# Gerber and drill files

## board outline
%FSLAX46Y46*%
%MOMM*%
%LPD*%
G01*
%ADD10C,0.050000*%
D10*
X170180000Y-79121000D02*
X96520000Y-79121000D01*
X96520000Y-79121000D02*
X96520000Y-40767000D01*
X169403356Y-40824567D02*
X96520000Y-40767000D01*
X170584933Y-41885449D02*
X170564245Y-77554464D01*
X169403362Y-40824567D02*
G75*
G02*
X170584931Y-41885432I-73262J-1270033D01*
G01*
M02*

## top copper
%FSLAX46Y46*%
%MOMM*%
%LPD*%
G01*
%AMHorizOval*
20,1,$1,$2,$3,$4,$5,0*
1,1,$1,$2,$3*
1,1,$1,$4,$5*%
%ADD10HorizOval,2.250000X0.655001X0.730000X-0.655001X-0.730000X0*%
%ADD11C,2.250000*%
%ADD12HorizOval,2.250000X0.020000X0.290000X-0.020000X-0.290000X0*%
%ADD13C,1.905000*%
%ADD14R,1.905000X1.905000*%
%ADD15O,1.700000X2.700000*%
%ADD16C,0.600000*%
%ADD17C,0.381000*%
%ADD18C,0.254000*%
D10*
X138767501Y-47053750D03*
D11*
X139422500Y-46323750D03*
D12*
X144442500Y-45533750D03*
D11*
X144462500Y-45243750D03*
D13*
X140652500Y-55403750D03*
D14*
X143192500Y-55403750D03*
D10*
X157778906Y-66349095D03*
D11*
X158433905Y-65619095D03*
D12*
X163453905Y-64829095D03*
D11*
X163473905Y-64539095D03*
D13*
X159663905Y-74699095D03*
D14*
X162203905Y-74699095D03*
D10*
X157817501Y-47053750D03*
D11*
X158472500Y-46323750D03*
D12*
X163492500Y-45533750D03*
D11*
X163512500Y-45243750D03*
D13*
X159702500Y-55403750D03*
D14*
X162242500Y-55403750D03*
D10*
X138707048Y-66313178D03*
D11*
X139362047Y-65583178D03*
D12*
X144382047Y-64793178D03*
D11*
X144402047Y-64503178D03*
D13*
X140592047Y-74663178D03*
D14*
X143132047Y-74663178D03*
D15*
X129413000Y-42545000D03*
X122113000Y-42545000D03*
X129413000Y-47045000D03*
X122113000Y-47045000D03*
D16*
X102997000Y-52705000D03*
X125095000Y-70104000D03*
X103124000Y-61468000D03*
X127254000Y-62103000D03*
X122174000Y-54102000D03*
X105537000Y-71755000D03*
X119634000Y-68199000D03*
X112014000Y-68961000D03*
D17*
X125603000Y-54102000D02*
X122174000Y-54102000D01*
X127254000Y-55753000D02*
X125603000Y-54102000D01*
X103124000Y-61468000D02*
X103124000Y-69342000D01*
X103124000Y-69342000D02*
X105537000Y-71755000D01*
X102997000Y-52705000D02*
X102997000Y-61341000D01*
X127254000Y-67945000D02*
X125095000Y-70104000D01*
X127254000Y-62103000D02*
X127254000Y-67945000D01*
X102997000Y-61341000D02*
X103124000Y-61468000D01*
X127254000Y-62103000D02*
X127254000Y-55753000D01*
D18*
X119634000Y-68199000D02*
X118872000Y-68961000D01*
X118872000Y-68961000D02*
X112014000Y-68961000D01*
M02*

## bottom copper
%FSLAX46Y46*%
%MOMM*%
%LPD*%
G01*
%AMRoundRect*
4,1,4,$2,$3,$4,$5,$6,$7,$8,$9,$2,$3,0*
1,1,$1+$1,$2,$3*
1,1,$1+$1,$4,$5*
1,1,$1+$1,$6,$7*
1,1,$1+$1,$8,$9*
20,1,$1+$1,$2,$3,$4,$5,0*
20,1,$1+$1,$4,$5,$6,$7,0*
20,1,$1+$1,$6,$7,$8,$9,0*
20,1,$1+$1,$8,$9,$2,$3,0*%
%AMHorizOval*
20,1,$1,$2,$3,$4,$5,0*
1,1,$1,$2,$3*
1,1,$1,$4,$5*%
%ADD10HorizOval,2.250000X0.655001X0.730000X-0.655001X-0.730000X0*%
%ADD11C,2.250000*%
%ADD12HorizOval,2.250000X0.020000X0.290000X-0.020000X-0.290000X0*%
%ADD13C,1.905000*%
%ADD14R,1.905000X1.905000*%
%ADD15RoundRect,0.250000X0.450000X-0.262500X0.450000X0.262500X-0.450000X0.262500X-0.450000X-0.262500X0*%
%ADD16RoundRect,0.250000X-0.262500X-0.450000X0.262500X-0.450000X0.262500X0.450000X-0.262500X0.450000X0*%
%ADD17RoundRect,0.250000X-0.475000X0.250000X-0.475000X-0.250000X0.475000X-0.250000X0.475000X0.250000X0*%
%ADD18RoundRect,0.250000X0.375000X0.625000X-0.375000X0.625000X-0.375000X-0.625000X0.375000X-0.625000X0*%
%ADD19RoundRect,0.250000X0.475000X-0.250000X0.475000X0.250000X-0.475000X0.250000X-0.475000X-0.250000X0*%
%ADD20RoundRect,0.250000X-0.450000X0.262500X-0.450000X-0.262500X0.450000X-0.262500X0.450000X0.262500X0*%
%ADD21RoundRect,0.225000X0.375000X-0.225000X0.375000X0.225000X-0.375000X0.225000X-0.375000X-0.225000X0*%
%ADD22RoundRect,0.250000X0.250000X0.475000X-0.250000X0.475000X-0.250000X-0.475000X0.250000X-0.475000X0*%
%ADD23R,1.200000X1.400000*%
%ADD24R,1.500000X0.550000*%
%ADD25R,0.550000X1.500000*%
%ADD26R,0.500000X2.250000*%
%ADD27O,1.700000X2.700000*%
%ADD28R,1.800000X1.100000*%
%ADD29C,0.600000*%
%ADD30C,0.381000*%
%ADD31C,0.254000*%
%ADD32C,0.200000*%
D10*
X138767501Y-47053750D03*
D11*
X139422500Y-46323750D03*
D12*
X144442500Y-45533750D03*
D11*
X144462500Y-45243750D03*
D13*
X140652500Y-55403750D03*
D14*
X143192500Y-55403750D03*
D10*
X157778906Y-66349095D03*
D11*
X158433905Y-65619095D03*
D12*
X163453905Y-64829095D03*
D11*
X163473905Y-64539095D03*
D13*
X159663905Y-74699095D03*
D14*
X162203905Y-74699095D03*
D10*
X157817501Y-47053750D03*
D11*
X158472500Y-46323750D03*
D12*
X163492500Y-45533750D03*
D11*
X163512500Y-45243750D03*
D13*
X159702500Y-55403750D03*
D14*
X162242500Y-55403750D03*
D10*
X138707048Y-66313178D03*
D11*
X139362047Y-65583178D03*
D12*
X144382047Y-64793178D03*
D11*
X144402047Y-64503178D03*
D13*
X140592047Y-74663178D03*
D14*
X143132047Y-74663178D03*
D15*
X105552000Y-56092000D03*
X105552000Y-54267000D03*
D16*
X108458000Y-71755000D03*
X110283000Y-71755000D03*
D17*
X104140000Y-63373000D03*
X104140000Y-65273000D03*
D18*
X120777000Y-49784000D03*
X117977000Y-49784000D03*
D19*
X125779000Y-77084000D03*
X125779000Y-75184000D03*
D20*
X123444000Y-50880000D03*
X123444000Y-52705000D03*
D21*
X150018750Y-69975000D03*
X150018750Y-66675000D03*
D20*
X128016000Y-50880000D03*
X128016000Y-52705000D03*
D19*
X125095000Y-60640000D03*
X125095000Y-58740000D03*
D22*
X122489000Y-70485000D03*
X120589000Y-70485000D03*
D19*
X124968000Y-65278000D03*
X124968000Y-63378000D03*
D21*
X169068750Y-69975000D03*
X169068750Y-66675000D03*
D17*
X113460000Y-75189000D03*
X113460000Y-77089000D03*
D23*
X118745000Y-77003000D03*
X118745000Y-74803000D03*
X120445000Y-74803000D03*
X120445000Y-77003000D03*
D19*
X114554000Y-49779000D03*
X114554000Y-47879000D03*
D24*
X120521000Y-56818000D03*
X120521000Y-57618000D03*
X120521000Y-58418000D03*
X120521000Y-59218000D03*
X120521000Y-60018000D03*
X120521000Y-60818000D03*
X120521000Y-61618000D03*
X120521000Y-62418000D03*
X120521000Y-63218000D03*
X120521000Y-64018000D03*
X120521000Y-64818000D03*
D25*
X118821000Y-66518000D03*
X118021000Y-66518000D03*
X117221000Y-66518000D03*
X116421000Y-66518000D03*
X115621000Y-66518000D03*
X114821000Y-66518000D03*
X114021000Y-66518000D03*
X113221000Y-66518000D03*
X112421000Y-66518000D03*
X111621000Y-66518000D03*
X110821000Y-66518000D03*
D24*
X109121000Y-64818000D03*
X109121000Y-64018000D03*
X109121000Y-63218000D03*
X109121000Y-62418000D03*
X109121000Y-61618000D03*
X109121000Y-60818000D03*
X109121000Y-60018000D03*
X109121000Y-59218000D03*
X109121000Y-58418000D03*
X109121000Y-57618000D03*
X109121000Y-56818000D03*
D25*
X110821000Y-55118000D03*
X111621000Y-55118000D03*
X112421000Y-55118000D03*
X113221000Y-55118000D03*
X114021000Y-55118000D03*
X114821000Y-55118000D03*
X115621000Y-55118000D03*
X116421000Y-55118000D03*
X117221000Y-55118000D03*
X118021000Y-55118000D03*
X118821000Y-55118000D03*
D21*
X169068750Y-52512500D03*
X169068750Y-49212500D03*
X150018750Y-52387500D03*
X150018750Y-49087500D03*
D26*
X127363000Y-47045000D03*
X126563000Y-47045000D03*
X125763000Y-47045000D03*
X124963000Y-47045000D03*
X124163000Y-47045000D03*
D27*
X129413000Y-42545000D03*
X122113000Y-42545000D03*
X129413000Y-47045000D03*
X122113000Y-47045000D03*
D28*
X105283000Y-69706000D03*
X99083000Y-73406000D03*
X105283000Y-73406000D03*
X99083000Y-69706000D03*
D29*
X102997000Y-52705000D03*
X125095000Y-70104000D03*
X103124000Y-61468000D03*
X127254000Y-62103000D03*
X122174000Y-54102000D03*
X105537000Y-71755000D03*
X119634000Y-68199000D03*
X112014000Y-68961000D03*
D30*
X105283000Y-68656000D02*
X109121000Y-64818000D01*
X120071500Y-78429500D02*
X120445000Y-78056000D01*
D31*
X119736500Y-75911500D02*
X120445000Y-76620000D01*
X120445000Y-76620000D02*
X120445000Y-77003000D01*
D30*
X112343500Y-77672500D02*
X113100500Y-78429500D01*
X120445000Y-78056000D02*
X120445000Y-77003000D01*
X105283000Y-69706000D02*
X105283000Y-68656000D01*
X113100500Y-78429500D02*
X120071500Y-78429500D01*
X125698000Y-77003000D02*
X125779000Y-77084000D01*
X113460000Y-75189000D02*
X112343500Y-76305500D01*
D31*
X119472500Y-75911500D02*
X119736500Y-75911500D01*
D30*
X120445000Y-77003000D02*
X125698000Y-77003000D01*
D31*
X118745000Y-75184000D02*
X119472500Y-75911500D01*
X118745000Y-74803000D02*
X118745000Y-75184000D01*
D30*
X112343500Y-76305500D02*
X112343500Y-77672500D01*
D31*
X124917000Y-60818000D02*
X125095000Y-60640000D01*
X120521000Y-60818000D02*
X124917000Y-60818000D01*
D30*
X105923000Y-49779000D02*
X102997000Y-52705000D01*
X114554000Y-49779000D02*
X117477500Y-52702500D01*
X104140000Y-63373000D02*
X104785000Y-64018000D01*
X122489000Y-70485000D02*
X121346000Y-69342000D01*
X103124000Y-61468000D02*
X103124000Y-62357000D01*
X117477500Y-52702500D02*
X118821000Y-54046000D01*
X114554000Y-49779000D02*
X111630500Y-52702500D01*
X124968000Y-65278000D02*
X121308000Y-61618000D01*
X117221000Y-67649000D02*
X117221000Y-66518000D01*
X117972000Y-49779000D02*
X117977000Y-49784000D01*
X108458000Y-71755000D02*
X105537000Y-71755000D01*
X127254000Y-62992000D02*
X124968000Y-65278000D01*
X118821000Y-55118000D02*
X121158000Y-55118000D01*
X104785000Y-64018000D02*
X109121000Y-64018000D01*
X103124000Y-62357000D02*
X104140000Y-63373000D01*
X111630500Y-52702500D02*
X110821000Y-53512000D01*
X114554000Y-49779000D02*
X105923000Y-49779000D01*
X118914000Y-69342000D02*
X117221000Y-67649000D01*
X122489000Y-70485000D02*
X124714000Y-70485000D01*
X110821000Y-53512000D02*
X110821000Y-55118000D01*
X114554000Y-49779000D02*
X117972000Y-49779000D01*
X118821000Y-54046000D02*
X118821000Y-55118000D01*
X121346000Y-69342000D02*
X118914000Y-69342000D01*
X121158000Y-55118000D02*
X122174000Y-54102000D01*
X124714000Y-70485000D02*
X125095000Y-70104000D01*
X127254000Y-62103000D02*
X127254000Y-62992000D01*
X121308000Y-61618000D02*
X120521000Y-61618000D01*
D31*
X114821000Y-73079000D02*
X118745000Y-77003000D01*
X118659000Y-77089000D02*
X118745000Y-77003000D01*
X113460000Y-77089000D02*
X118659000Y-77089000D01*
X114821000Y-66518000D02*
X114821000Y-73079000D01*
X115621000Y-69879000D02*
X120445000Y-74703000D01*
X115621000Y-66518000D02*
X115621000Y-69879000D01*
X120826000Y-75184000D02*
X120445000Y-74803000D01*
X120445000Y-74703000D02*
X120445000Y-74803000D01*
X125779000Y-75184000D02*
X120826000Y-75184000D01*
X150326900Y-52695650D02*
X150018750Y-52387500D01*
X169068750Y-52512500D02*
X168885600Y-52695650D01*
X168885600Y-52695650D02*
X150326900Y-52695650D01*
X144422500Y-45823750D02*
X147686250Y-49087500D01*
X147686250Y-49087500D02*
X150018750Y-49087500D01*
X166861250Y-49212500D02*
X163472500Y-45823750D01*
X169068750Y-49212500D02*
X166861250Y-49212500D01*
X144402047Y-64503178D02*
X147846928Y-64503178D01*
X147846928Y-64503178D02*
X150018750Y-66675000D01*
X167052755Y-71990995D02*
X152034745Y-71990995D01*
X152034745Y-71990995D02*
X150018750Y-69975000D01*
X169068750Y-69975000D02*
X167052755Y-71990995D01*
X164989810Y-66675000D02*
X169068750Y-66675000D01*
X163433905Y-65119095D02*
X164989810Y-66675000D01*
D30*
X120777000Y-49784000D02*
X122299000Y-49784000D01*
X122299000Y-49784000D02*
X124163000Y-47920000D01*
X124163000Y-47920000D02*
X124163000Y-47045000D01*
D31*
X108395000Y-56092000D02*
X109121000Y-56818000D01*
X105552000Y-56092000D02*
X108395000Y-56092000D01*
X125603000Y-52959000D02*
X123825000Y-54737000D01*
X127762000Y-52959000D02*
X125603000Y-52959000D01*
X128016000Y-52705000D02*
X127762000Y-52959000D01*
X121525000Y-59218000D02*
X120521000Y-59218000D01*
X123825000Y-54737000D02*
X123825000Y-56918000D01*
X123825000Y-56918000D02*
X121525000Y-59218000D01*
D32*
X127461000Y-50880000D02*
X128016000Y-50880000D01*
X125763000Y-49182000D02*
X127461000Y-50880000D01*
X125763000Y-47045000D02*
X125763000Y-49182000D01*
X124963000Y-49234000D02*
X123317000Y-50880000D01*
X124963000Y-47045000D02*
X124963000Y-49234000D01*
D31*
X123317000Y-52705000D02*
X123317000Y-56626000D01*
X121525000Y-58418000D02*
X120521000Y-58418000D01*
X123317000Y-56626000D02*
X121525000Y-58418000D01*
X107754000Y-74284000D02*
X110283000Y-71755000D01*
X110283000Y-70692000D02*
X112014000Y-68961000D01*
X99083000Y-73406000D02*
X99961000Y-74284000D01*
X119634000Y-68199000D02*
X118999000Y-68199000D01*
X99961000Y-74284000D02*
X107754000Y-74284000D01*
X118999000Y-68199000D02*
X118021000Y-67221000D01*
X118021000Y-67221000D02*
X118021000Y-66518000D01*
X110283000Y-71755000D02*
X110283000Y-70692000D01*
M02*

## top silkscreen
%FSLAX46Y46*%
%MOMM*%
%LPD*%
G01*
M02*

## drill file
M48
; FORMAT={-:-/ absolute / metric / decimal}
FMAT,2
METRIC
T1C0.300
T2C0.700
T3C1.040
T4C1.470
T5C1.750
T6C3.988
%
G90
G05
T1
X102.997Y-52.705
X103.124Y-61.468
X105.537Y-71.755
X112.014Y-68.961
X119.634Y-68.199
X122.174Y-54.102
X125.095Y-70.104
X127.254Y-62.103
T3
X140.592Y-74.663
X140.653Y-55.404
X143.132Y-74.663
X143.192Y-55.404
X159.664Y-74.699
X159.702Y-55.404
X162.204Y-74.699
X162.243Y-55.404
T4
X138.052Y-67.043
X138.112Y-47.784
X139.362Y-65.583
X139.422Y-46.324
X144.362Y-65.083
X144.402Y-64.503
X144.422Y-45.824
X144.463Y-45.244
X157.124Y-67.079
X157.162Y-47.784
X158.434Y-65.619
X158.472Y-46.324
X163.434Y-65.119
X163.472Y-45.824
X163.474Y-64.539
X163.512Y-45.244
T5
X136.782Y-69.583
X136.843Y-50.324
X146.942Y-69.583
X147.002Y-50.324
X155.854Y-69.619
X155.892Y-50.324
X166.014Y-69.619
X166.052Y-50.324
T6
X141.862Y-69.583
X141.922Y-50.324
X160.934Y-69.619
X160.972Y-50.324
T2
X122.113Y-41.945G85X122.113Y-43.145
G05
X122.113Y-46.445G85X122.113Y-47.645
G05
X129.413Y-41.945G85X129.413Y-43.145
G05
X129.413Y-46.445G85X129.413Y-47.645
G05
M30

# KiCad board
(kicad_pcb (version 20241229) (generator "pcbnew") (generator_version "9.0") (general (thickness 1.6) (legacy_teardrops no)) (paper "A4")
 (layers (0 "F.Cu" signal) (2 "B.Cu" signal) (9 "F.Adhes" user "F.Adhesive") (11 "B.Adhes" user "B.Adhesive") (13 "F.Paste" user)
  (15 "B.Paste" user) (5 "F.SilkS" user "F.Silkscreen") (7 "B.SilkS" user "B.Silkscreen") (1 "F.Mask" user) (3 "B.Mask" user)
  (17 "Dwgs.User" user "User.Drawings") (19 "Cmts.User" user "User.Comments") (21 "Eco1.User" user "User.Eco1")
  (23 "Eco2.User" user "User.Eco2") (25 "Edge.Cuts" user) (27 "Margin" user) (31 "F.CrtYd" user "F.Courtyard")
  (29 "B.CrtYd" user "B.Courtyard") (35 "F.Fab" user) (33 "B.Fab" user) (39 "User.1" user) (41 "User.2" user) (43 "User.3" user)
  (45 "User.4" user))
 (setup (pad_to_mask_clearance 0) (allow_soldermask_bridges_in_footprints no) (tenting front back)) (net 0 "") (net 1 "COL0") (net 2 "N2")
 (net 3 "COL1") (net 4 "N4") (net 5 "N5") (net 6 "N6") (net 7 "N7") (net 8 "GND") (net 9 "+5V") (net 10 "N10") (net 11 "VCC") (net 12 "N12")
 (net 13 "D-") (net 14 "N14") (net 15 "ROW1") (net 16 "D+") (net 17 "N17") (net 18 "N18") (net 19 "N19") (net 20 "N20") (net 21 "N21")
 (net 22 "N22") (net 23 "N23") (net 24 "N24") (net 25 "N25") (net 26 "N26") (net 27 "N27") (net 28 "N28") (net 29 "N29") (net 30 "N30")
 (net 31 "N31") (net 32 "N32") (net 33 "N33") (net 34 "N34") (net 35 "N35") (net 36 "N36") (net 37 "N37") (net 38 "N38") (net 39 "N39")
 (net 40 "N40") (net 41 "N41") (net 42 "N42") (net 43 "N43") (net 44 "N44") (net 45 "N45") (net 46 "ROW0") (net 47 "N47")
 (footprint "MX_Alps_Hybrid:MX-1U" (layer "F.Cu") (at 141.9225 50.32375)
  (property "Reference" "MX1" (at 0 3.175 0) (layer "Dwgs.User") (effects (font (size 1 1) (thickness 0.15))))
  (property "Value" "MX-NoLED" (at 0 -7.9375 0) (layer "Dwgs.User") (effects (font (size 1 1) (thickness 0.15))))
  (pad "" np_thru_hole circle (at -5.08 0 48.0996) (size 1.75 1.75) (drill 1.75) (layers "*.Cu" "*.Mask"))
  (pad "" np_thru_hole circle (at 0 0) (size 3.9878 3.9878) (drill 3.9878) (layers "*.Cu" "*.Mask"))
  (pad "" np_thru_hole circle (at 5.08 0 48.0996) (size 1.75 1.75) (drill 1.75) (layers "*.Cu" "*.Mask"))
  (pad "1" thru_hole oval (at -3.81 -2.54 48.0996) (size 4.211556 2.25) (drill 1.47 (offset 0.980778 0)) (layers "*.Cu" "B.Mask")
   (remove_unused_layers no) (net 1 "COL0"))
  (pad "1" thru_hole circle (at -2.5 -4) (size 2.25 2.25) (drill 1.47) (layers "*.Cu" "B.Mask") (remove_unused_layers no) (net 1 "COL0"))
  (pad "2" thru_hole oval (at 2.5 -4.5 86.0548) (size 2.831378 2.25) (drill 1.47 (offset 0.290689 0)) (layers "*.Cu" "B.Mask")
   (remove_unused_layers no) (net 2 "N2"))
  (pad "2" thru_hole circle (at 2.54 -5.08) (size 2.25 2.25) (drill 1.47) (layers "*.Cu" "B.Mask") (remove_unused_layers no) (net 2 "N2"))
  (pad "3" thru_hole circle (at -1.27 5.08) (size 1.905 1.905) (drill 1.04) (layers "*.Cu" "B.Mask") (remove_unused_layers no))
  (pad "4" thru_hole rect (at 1.27 5.08) (size 1.905 1.905) (drill 1.04) (layers "*.Cu" "B.Mask") (remove_unused_layers no)))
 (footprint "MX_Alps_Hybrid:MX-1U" (layer "F.Cu") (at 160.933905 69.619095)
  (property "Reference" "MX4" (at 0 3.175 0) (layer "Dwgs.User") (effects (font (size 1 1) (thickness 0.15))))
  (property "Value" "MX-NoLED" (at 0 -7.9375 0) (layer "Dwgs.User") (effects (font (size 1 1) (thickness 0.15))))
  (pad "" np_thru_hole circle (at -5.08 0 48.0996) (size 1.75 1.75) (drill 1.75) (layers "*.Cu" "*.Mask"))
  (pad "" np_thru_hole circle (at 0 0) (size 3.9878 3.9878) (drill 3.9878) (layers "*.Cu" "*.Mask"))
  (pad "" np_thru_hole circle (at 5.08 0 48.0996) (size 1.75 1.75) (drill 1.75) (layers "*.Cu" "*.Mask"))
  (pad "1" thru_hole oval (at -3.81 -2.54 48.0996) (size 4.211556 2.25) (drill 1.47 (offset 0.980778 0)) (layers "*.Cu" "B.Mask")
   (remove_unused_layers no) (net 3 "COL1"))
  (pad "1" thru_hole circle (at -2.5 -4) (size 2.25 2.25) (drill 1.47) (layers "*.Cu" "B.Mask") (remove_unused_layers no) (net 3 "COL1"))
  (pad "2" thru_hole oval (at 2.5 -4.5 86.0548) (size 2.831378 2.25) (drill 1.47 (offset 0.290689 0)) (layers "*.Cu" "B.Mask")
   (remove_unused_layers no) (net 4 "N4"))
  (pad "2" thru_hole circle (at 2.54 -5.08) (size 2.25 2.25) (drill 1.47) (layers "*.Cu" "B.Mask") (remove_unused_layers no) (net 4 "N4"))
  (pad "3" thru_hole circle (at -1.27 5.08) (size 1.905 1.905) (drill 1.04) (layers "*.Cu" "B.Mask") (remove_unused_layers no))
  (pad "4" thru_hole rect (at 1.27 5.08) (size 1.905 1.905) (drill 1.04) (layers "*.Cu" "B.Mask") (remove_unused_layers no)))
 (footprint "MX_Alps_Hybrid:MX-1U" (layer "F.Cu") (at 160.9725 50.32375)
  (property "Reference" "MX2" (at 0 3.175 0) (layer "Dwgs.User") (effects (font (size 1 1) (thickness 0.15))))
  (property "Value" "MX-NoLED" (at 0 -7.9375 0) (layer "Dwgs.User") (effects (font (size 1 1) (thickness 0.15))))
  (pad "" np_thru_hole circle (at -5.08 0 48.0996) (size 1.75 1.75) (drill 1.75) (layers "*.Cu" "*.Mask"))
  (pad "" np_thru_hole circle (at 0 0) (size 3.9878 3.9878) (drill 3.9878) (layers "*.Cu" "*.Mask"))
  (pad "" np_thru_hole circle (at 5.08 0 48.0996) (size 1.75 1.75) (drill 1.75) (layers "*.Cu" "*.Mask"))
  (pad "1" thru_hole oval (at -3.81 -2.54 48.0996) (size 4.211556 2.25) (drill 1.47 (offset 0.980778 0)) (layers "*.Cu" "B.Mask")
   (remove_unused_layers no) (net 3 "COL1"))
  (pad "1" thru_hole circle (at -2.5 -4) (size 2.25 2.25) (drill 1.47) (layers "*.Cu" "B.Mask") (remove_unused_layers no) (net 3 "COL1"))
  (pad "2" thru_hole oval (at 2.5 -4.5 86.0548) (size 2.831378 2.25) (drill 1.47 (offset 0.290689 0)) (layers "*.Cu" "B.Mask")
   (remove_unused_layers no) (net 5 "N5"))
  (pad "2" thru_hole circle (at 2.54 -5.08) (size 2.25 2.25) (drill 1.47) (layers "*.Cu" "B.Mask") (remove_unused_layers no) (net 5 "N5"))
  (pad "3" thru_hole circle (at -1.27 5.08) (size 1.905 1.905) (drill 1.04) (layers "*.Cu" "B.Mask") (remove_unused_layers no))
  (pad "4" thru_hole rect (at 1.27 5.08) (size 1.905 1.905) (drill 1.04) (layers "*.Cu" "B.Mask") (remove_unused_layers no)))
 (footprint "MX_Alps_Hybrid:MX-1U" (layer "F.Cu") (at 141.862047 69.583178)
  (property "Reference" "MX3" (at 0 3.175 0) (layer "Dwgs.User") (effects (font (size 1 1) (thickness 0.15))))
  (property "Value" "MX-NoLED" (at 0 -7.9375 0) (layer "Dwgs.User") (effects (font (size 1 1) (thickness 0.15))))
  (pad "" np_thru_hole circle (at -5.08 0 48.0996) (size 1.75 1.75) (drill 1.75) (layers "*.Cu" "*.Mask"))
  (pad "" np_thru_hole circle (at 0 0) (size 3.9878 3.9878) (drill 3.9878) (layers "*.Cu" "*.Mask"))
  (pad "" np_thru_hole circle (at 5.08 0 48.0996) (size 1.75 1.75) (drill 1.75) (layers "*.Cu" "*.Mask"))
  (pad "1" thru_hole oval (at -3.81 -2.54 48.0996) (size 4.211556 2.25) (drill 1.47 (offset 0.980778 0)) (layers "*.Cu" "B.Mask")
   (remove_unused_layers no) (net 1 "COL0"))
  (pad "1" thru_hole circle (at -2.5 -4) (size 2.25 2.25) (drill 1.47) (layers "*.Cu" "B.Mask") (remove_unused_layers no) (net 1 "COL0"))
  (pad "2" thru_hole oval (at 2.5 -4.5 86.0548) (size 2.831378 2.25) (drill 1.47 (offset 0.290689 0)) (layers "*.Cu" "B.Mask")
   (remove_unused_layers no) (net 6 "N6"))
  (pad "2" thru_hole circle (at 2.54 -5.08) (size 2.25 2.25) (drill 1.47) (layers "*.Cu" "B.Mask") (remove_unused_layers no) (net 6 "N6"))
  (pad "3" thru_hole circle (at -1.27 5.08) (size 1.905 1.905) (drill 1.04) (layers "*.Cu" "B.Mask") (remove_unused_layers no))
  (pad "4" thru_hole rect (at 1.27 5.08) (size 1.905 1.905) (drill 1.04) (layers "*.Cu" "B.Mask") (remove_unused_layers no)))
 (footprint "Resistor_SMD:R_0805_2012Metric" (layer "B.Cu") (at 105.552 55.1795 90)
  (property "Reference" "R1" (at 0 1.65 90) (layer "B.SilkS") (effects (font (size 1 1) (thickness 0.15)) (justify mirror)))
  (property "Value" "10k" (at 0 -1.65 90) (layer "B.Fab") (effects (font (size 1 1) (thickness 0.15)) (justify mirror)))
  (pad "1" smd roundrect (at -0.9125 0 90) (size 1.025 1.4) (layers "B.Cu" "B.Mask" "B.Paste") (roundrect_rratio 0.243902) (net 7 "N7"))
  (pad "2" smd roundrect (at 0.9125 0 90) (size 1.025 1.4) (layers "B.Cu" "B.Mask" "B.Paste") (roundrect_rratio 0.243902) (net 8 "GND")))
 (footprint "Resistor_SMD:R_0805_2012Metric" (layer "B.Cu") (at 109.3705 71.755)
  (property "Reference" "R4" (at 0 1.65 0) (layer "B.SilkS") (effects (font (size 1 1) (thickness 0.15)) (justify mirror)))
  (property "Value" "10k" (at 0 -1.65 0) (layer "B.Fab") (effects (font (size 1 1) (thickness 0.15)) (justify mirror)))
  (pad "1" smd roundrect (at -0.9125 0) (size 1.025 1.4) (layers "B.Cu" "B.Mask" "B.Paste") (roundrect_rratio 0.243902) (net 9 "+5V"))
  (pad "2" smd roundrect (at 0.9125 0) (size 1.025 1.4) (layers "B.Cu" "B.Mask" "B.Paste") (roundrect_rratio 0.243902) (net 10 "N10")))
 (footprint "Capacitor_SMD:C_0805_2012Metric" (layer "B.Cu") (at 104.14 64.323 -90)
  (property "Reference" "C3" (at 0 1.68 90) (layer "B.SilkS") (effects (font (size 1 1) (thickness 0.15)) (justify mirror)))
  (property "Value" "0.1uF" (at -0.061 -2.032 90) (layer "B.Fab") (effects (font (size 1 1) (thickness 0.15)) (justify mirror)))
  (pad "1" smd roundrect (at -0.95 0 270) (size 1 1.45) (layers "B.Cu" "B.Mask" "B.Paste") (roundrect_rratio 0.25) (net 9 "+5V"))
  (pad "2" smd roundrect (at 0.95 0 270) (size 1 1.45) (layers "B.Cu" "B.Mask" "B.Paste") (roundrect_rratio 0.25) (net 8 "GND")))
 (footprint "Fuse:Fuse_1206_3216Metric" (layer "B.Cu") (at 119.377 49.784 180)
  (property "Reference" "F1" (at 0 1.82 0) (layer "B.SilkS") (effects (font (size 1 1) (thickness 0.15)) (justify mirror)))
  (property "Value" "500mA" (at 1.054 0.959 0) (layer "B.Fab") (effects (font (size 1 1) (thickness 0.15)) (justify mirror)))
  (pad "1" smd roundrect (at -1.4 0 180) (size 1.25 1.75) (layers "B.Cu" "B.Mask" "B.Paste") (roundrect_rratio 0.2) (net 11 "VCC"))
  (pad "2" smd roundrect (at 1.4 0 180) (size 1.25 1.75) (layers "B.Cu" "B.Mask" "B.Paste") (roundrect_rratio 0.2) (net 9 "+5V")))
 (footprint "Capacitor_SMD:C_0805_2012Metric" (layer "B.Cu") (at 125.779 76.134 90)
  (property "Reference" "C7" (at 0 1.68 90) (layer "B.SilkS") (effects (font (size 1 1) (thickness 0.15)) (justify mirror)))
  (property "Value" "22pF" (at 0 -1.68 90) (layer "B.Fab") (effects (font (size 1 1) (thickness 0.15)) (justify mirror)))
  (pad "1" smd roundrect (at -0.95 0 90) (size 1 1.45) (layers "B.Cu" "B.Mask" "B.Paste") (roundrect_rratio 0.25) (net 8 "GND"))
  (pad "2" smd roundrect (at 0.95 0 90) (size 1 1.45) (layers "B.Cu" "B.Mask" "B.Paste") (roundrect_rratio 0.25) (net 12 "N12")))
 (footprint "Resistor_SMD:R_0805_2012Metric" (layer "B.Cu") (at 123.444 51.7925 -90)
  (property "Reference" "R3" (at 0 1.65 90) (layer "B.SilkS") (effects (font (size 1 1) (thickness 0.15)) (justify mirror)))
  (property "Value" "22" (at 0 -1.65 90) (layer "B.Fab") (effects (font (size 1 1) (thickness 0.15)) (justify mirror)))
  (pad "1" smd roundrect (at -0.9125 0 270) (size 1.025 1.4) (layers "B.Cu" "B.Mask" "B.Paste") (roundrect_rratio 0.243902) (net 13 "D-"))
  (pad "2" smd roundrect (at 0.9125 0 270) (size 1.025 1.4) (layers "B.Cu" "B.Mask" "B.Paste") (roundrect_rratio 0.243902) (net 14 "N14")))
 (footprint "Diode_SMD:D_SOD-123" (layer "B.Cu") (at 150.01875 68.325 90)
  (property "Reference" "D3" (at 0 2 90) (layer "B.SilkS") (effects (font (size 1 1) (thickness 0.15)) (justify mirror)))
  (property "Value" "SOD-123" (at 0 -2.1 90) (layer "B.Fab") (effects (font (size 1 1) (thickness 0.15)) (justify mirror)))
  (pad "1" smd roundrect (at -1.65 0 90) (size 0.9 1.2) (layers "B.Cu" "B.Mask" "B.Paste") (roundrect_rratio 0.25) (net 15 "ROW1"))
  (pad "2" smd roundrect (at 1.65 0 90) (size 0.9 1.2) (layers "B.Cu" "B.Mask" "B.Paste") (roundrect_rratio 0.25) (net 6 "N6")))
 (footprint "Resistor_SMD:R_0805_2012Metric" (layer "B.Cu") (at 128.016 51.7925 -90)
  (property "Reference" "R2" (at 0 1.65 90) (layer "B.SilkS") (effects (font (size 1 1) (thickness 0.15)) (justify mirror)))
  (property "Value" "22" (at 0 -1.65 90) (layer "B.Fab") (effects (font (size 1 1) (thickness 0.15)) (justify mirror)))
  (pad "1" smd roundrect (at -0.9125 0 270) (size 1.025 1.4) (layers "B.Cu" "B.Mask" "B.Paste") (roundrect_rratio 0.243902) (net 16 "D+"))
  (pad "2" smd roundrect (at 0.9125 0 270) (size 1.025 1.4) (layers "B.Cu" "B.Mask" "B.Paste") (roundrect_rratio 0.243902) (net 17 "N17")))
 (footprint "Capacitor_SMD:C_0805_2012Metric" (layer "B.Cu") (at 125.095 59.69 90)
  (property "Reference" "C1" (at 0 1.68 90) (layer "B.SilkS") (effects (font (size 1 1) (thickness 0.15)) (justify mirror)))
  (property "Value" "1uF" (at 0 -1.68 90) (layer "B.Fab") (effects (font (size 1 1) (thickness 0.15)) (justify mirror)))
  (pad "1" smd roundrect (at -0.95 0 90) (size 1 1.45) (layers "B.Cu" "B.Mask" "B.Paste") (roundrect_rratio 0.25) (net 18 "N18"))
  (pad "2" smd roundrect (at 0.95 0 90) (size 1 1.45) (layers "B.Cu" "B.Mask" "B.Paste") (roundrect_rratio 0.25) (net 8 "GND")))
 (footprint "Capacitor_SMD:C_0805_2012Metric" (layer "B.Cu") (at 121.539 70.485 180)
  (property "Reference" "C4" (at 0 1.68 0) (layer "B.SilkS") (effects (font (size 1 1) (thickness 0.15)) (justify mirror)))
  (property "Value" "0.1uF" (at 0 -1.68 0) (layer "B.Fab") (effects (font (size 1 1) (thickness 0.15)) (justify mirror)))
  (pad "1" smd roundrect (at -0.95 0 180) (size 1 1.45) (layers "B.Cu" "B.Mask" "B.Paste") (roundrect_rratio 0.25) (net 9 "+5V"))
  (pad "2" smd roundrect (at 0.95 0 180) (size 1 1.45) (layers "B.Cu" "B.Mask" "B.Paste") (roundrect_rratio 0.25) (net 8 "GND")))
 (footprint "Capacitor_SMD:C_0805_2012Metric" (layer "B.Cu") (at 124.968 64.328 90)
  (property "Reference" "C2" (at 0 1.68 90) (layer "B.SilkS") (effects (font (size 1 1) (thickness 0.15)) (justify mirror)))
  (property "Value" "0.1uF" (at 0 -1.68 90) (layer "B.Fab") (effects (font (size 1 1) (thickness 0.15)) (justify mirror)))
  (pad "1" smd roundrect (at -0.95 0 90) (size 1 1.45) (layers "B.Cu" "B.Mask" "B.Paste") (roundrect_rratio 0.25) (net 9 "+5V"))
  (pad "2" smd roundrect (at 0.95 0 90) (size 1 1.45) (layers "B.Cu" "B.Mask" "B.Paste") (roundrect_rratio 0.25) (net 8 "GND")))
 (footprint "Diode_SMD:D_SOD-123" (layer "B.Cu") (at 169.06875 68.325 90)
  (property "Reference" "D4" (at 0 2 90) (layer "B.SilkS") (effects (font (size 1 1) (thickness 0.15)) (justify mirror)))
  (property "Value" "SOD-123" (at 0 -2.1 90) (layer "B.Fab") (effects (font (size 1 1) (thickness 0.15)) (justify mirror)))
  (pad "1" smd roundrect (at -1.65 0 90) (size 0.9 1.2) (layers "B.Cu" "B.Mask" "B.Paste") (roundrect_rratio 0.25) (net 15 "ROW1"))
  (pad "2" smd roundrect (at 1.65 0 90) (size 0.9 1.2) (layers "B.Cu" "B.Mask" "B.Paste") (roundrect_rratio 0.25) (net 4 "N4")))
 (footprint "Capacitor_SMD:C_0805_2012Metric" (layer "B.Cu") (at 113.46 76.139 -90)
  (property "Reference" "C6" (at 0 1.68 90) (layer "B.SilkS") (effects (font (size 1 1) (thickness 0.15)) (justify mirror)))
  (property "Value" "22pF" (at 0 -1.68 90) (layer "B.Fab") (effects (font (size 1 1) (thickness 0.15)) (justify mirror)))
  (pad "1" smd roundrect (at -0.95 0 270) (size 1 1.45) (layers "B.Cu" "B.Mask" "B.Paste") (roundrect_rratio 0.25) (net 8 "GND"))
  (pad "2" smd roundrect (at 0.95 0 270) (size 1 1.45) (layers "B.Cu" "B.Mask" "B.Paste") (roundrect_rratio 0.25) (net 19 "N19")))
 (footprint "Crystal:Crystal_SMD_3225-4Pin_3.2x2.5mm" (layer "B.Cu") (at 119.595 75.903 90)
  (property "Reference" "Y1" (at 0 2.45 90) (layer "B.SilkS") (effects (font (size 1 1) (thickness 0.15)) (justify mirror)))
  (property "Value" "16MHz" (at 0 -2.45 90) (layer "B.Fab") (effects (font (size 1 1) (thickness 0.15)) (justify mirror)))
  (pad "1" smd rect (at -1.1 -0.85 90) (size 1.4 1.2) (layers "B.Cu" "B.Mask" "B.Paste") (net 19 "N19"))
  (pad "2" smd rect (at 1.1 -0.85 90) (size 1.4 1.2) (layers "B.Cu" "B.Mask" "B.Paste") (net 8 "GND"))
  (pad "3" smd rect (at 1.1 0.85 90) (size 1.4 1.2) (layers "B.Cu" "B.Mask" "B.Paste") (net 12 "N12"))
  (pad "4" smd rect (at -1.1 0.85 90) (size 1.4 1.2) (layers "B.Cu" "B.Mask" "B.Paste") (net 8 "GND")))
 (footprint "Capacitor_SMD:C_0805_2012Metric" (layer "B.Cu") (at 114.554 48.829 90)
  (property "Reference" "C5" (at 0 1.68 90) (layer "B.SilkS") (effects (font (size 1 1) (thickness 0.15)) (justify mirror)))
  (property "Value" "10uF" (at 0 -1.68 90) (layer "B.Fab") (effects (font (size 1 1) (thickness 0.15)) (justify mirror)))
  (pad "1" smd roundrect (at -0.95 0 90) (size 1 1.45) (layers "B.Cu" "B.Mask" "B.Paste") (roundrect_rratio 0.25) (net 9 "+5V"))
  (pad "2" smd roundrect (at 0.95 0 90) (size 1 1.45) (layers "B.Cu" "B.Mask" "B.Paste") (roundrect_rratio 0.25) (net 8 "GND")))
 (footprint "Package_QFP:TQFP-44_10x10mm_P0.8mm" (layer "B.Cu") (at 114.821 60.818 180)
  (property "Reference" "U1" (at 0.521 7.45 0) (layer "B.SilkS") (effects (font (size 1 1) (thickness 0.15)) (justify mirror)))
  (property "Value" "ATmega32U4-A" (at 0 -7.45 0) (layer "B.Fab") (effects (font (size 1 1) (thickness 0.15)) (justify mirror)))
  (pad "1" smd rect (at -5.7 4 180) (size 1.5 0.55) (layers "B.Cu" "B.Mask" "B.Paste") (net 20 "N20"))
  (pad "2" smd rect (at -5.7 3.2 180) (size 1.5 0.55) (layers "B.Cu" "B.Mask" "B.Paste") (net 9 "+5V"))
  (pad "3" smd rect (at -5.7 2.4 180) (size 1.5 0.55) (layers "B.Cu" "B.Mask" "B.Paste") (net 14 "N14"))
  (pad "4" smd rect (at -5.7 1.6 180) (size 1.5 0.55) (layers "B.Cu" "B.Mask" "B.Paste") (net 17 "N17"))
  (pad "5" smd rect (at -5.7 0.8 180) (size 1.5 0.55) (layers "B.Cu" "B.Mask" "B.Paste") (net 8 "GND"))
  (pad "6" smd rect (at -5.7 0 180) (size 1.5 0.55) (layers "B.Cu" "B.Mask" "B.Paste") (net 18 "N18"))
  (pad "7" smd rect (at -5.7 -0.8 180) (size 1.5 0.55) (layers "B.Cu" "B.Mask" "B.Paste") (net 9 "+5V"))
  (pad "8" smd rect (at -5.7 -1.6 180) (size 1.5 0.55) (layers "B.Cu" "B.Mask" "B.Paste") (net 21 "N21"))
  (pad "9" smd rect (at -5.7 -2.4 180) (size 1.5 0.55) (layers "B.Cu" "B.Mask" "B.Paste") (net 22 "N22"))
  (pad "10" smd rect (at -5.7 -3.2 180) (size 1.5 0.55) (layers "B.Cu" "B.Mask" "B.Paste") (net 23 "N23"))
  (pad "11" smd rect (at -5.7 -4 180) (size 1.5 0.55) (layers "B.Cu" "B.Mask" "B.Paste") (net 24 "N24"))
  (pad "12" smd rect (at -4 -5.7 90) (size 1.5 0.55) (layers "B.Cu" "B.Mask" "B.Paste") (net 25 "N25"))
  (pad "13" smd rect (at -3.2 -5.7 90) (size 1.5 0.55) (layers "B.Cu" "B.Mask" "B.Paste") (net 10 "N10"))
  (pad "14" smd rect (at -2.4 -5.7 90) (size 1.5 0.55) (layers "B.Cu" "B.Mask" "B.Paste") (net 9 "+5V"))
  (pad "15" smd rect (at -1.6 -5.7 90) (size 1.5 0.55) (layers "B.Cu" "B.Mask" "B.Paste") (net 8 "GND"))
  (pad "16" smd rect (at -0.8 -5.7 90) (size 1.5 0.55) (layers "B.Cu" "B.Mask" "B.Paste") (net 12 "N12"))
  (pad "17" smd rect (at 0 -5.7 90) (size 1.5 0.55) (layers "B.Cu" "B.Mask" "B.Paste") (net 19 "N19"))
  (pad "18" smd rect (at 0.8 -5.7 90) (size 1.5 0.55) (layers "B.Cu" "B.Mask" "B.Paste") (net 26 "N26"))
  (pad "19" smd rect (at 1.6 -5.7 90) (size 1.5 0.55) (layers "B.Cu" "B.Mask" "B.Paste") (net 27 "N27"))
  (pad "20" smd rect (at 2.4 -5.7 90) (size 1.5 0.55) (layers "B.Cu" "B.Mask" "B.Paste") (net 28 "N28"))
  (pad "21" smd rect (at 3.2 -5.7 90) (size 1.5 0.55) (layers "B.Cu" "B.Mask" "B.Paste") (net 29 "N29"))
  (pad "22" smd rect (at 4 -5.7 90) (size 1.5 0.55) (layers "B.Cu" "B.Mask" "B.Paste") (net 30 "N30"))
  (pad "23" smd rect (at 5.7 -4 180) (size 1.5 0.55) (layers "B.Cu" "B.Mask" "B.Paste") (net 8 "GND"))
  (pad "24" smd rect (at 5.7 -3.2 180) (size 1.5 0.55) (layers "B.Cu" "B.Mask" "B.Paste") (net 9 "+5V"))
  (pad "25" smd rect (at 5.7 -2.4 180) (size 1.5 0.55) (layers "B.Cu" "B.Mask" "B.Paste") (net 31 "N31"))
  (pad "26" smd rect (at 5.7 -1.6 180) (size 1.5 0.55) (layers "B.Cu" "B.Mask" "B.Paste") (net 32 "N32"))
  (pad "27" smd rect (at 5.7 -0.8 180) (size 1.5 0.55) (layers "B.Cu" "B.Mask" "B.Paste") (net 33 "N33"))
  (pad "28" smd rect (at 5.7 0 180) (size 1.5 0.55) (layers "B.Cu" "B.Mask" "B.Paste") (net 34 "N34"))
  (pad "29" smd rect (at 5.7 0.8 180) (size 1.5 0.55) (layers "B.Cu" "B.Mask" "B.Paste") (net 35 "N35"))
  (pad "30" smd rect (at 5.7 1.6 180) (size 1.5 0.55) (layers "B.Cu" "B.Mask" "B.Paste") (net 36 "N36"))
  (pad "31" smd rect (at 5.7 2.4 180) (size 1.5 0.55) (layers "B.Cu" "B.Mask" "B.Paste") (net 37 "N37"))
  (pad "32" smd rect (at 5.7 3.2 180) (size 1.5 0.55) (layers "B.Cu" "B.Mask" "B.Paste") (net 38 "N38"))
  (pad "33" smd rect (at 5.7 4 180) (size 1.5 0.55) (layers "B.Cu" "B.Mask" "B.Paste") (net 7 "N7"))
  (pad "34" smd rect (at 4 5.7 90) (size 1.5 0.55) (layers "B.Cu" "B.Mask" "B.Paste") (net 9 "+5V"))
  (pad "35" smd rect (at 3.2 5.7 90) (size 1.5 0.55) (layers "B.Cu" "B.Mask" "B.Paste") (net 8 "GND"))
  (pad "36" smd rect (at 2.4 5.7 90) (size 1.5 0.55) (layers "B.Cu" "B.Mask" "B.Paste") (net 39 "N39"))
  (pad "37" smd rect (at 1.6 5.7 90) (size 1.5 0.55) (layers "B.Cu" "B.Mask" "B.Paste") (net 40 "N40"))
  (pad "38" smd rect (at 0.8 5.7 90) (size 1.5 0.55) (layers "B.Cu" "B.Mask" "B.Paste") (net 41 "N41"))
  (pad "39" smd rect (at 0 5.7 90) (size 1.5 0.55) (layers "B.Cu" "B.Mask" "B.Paste") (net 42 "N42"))
  (pad "40" smd rect (at -0.8 5.7 90) (size 1.5 0.55) (layers "B.Cu" "B.Mask" "B.Paste") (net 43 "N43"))
  (pad "41" smd rect (at -1.6 5.7 90) (size 1.5 0.55) (layers "B.Cu" "B.Mask" "B.Paste") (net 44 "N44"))
  (pad "42" smd rect (at -2.4 5.7 90) (size 1.5 0.55) (layers "B.Cu" "B.Mask" "B.Paste") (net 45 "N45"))
  (pad "43" smd rect (at -3.2 5.7 90) (size 1.5 0.55) (layers "B.Cu" "B.Mask" "B.Paste") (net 8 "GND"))
  (pad "44" smd rect (at -4 5.7 90) (size 1.5 0.55) (layers "B.Cu" "B.Mask" "B.Paste") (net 9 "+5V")))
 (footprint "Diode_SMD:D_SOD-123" (layer "B.Cu") (at 169.06875 50.8625 90)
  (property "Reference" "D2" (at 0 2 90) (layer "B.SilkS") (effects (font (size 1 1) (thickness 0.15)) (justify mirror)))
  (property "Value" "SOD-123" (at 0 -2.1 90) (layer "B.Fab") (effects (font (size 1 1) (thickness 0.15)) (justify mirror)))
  (pad "1" smd roundrect (at -1.65 0 90) (size 0.9 1.2) (layers "B.Cu" "B.Mask" "B.Paste") (roundrect_rratio 0.25) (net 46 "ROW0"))
  (pad "2" smd roundrect (at 1.65 0 90) (size 0.9 1.2) (layers "B.Cu" "B.Mask" "B.Paste") (roundrect_rratio 0.25) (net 5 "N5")))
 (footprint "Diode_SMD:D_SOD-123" (layer "B.Cu") (at 150.01875 50.7375 90)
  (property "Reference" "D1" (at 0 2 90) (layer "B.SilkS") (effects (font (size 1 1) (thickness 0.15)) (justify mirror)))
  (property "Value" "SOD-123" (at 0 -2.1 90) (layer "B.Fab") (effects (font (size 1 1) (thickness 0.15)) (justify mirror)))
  (pad "1" smd roundrect (at -1.65 0 90) (size 0.9 1.2) (layers "B.Cu" "B.Mask" "B.Paste") (roundrect_rratio 0.25) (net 46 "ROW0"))
  (pad "2" smd roundrect (at 1.65 0 90) (size 0.9 1.2) (layers "B.Cu" "B.Mask" "B.Paste") (roundrect_rratio 0.25) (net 2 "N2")))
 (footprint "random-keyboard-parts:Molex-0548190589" (layer "B.Cu") (at 125.763 42.545 -90)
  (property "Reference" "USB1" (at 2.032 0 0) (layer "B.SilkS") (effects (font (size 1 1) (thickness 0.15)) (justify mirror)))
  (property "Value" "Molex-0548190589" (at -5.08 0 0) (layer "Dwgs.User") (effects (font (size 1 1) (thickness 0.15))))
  (pad "1" smd rect (at 4.5 -1.6 270) (size 2.25 0.5) (layers "B.Cu" "B.Mask" "B.Paste") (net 8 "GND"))
  (pad "2" smd rect (at 4.5 -0.8 270) (size 2.25 0.5) (layers "B.Cu" "B.Mask" "B.Paste") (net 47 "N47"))
  (pad "3" smd rect (at 4.5 0 270) (size 2.25 0.5) (layers "B.Cu" "B.Mask" "B.Paste") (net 16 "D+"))
  (pad "4" smd rect (at 4.5 0.8 270) (size 2.25 0.5) (layers "B.Cu" "B.Mask" "B.Paste") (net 13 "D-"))
  (pad "5" smd rect (at 4.5 1.6 270) (size 2.25 0.5) (layers "B.Cu" "B.Mask" "B.Paste") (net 11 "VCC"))
  (pad "6" thru_hole oval (at 0 -3.65 270) (size 2.7 1.7) (drill oval 1.9 0.7) (layers "*.Cu" "*.Mask") (remove_unused_layers no)
   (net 8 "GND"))
  (pad "6" thru_hole oval (at 0 3.65 270) (size 2.7 1.7) (drill oval 1.9 0.7) (layers "*.Cu" "*.Mask") (remove_unused_layers no)
   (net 8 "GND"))
  (pad "6" thru_hole oval (at 4.5 -3.65 270) (size 2.7 1.7) (drill oval 1.9 0.7) (layers "*.Cu" "*.Mask") (remove_unused_layers no)
   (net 8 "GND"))
  (pad "6" thru_hole oval (at 4.5 3.65 270) (size 2.7 1.7) (drill oval 1.9 0.7) (layers "*.Cu" "*.Mask") (remove_unused_layers no)
   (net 8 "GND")))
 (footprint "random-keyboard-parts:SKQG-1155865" (layer "B.Cu") (at 102.183 71.556)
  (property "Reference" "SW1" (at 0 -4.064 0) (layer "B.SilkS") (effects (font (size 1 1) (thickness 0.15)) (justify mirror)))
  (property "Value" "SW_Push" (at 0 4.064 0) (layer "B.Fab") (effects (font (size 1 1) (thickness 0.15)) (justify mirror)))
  (pad "1" smd rect (at 3.1 -1.85) (size 1.8 1.1) (layers "B.Cu" "B.Mask" "B.Paste") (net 8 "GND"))
  (pad "2" smd rect (at -3.1 1.85) (size 1.8 1.1) (layers "B.Cu" "B.Mask" "B.Paste") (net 10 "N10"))
  (pad "3" smd rect (at 3.1 1.85) (size 1.8 1.1) (layers "B.Cu" "B.Mask" "B.Paste"))
  (pad "4" smd rect (at -3.1 -1.85) (size 1.8 1.1) (layers "B.Cu" "B.Mask" "B.Paste")))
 (gr_line (start 170.18 79.121) (end 96.52 79.121) (stroke (width 0.05) (type default)) (layer "Edge.Cuts"))
 (gr_line (start 96.52 79.121) (end 96.52 40.767) (stroke (width 0.05) (type default)) (layer "Edge.Cuts"))
 (gr_line (start 169.403356 40.824567) (end 96.52 40.767) (stroke (width 0.05) (type default)) (layer "Edge.Cuts"))
 (gr_line (start 170.584933 41.885449) (end 170.564245 77.554464) (stroke (width 0.05) (type default)) (layer "Edge.Cuts"))
 (gr_arc (start 169.403362 40.824567) (mid 170.18 41.148) (end 170.584933 41.885432) (stroke (width 0.05) (type default))
  (layer "Edge.Cuts"))
 (segment (start 105.283 68.656) (end 109.121 64.818) (width 0.381) (layer "B.Cu") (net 8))
 (segment (start 120.0715 78.4295) (end 120.445 78.056) (width 0.381) (layer "B.Cu") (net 8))
 (segment (start 119.7365 75.9115) (end 120.445 76.62) (width 0.254) (layer "B.Cu") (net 8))
 (segment (start 120.445 76.62) (end 120.445 77.003) (width 0.254) (layer "B.Cu") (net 8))
 (segment (start 112.3435 77.6725) (end 113.1005 78.4295) (width 0.381) (layer "B.Cu") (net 8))
 (segment (start 120.445 78.056) (end 120.445 77.003) (width 0.381) (layer "B.Cu") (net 8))
 (segment (start 105.283 69.706) (end 105.283 68.656) (width 0.381) (layer "B.Cu") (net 8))
 (segment (start 113.1005 78.4295) (end 120.0715 78.4295) (width 0.381) (layer "B.Cu") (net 8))
 (segment (start 125.698 77.003) (end 125.779 77.084) (width 0.381) (layer "B.Cu") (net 8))
 (segment (start 113.46 75.189) (end 112.3435 76.3055) (width 0.381) (layer "B.Cu") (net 8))
 (segment (start 119.4725 75.9115) (end 119.7365 75.9115) (width 0.254) (layer "B.Cu") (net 8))
 (segment (start 120.445 77.003) (end 125.698 77.003) (width 0.381) (layer "B.Cu") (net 8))
 (segment (start 118.745 75.184) (end 119.4725 75.9115) (width 0.254) (layer "B.Cu") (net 8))
 (segment (start 118.745 74.803) (end 118.745 75.184) (width 0.254) (layer "B.Cu") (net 8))
 (segment (start 112.3435 76.3055) (end 112.3435 77.6725) (width 0.381) (layer "B.Cu") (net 8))
 (segment (start 124.917 60.818) (end 125.095 60.64) (width 0.254) (layer "B.Cu") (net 18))
 (segment (start 120.521 60.818) (end 124.917 60.818) (width 0.254) (layer "B.Cu") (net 18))
 (segment (start 125.603 54.102) (end 122.174 54.102) (width 0.381) (layer "F.Cu") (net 9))
 (segment (start 127.254 55.753) (end 125.603 54.102) (width 0.381) (layer "F.Cu") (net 9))
 (segment (start 103.124 61.468) (end 103.124 69.342) (width 0.381) (layer "F.Cu") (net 9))
 (segment (start 103.124 69.342) (end 105.537 71.755) (width 0.381) (layer "F.Cu") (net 9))
 (segment (start 102.997 52.705) (end 102.997 61.341) (width 0.381) (layer "F.Cu") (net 9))
 (segment (start 127.254 67.945) (end 125.095 70.104) (width 0.381) (layer "F.Cu") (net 9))
 (segment (start 127.254 62.103) (end 127.254 67.945) (width 0.381) (layer "F.Cu") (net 9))
 (segment (start 102.997 61.341) (end 103.124 61.468) (width 0.381) (layer "F.Cu") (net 9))
 (segment (start 127.254 62.103) (end 127.254 55.753) (width 0.381) (layer "F.Cu") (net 9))
 (via (at 102.997 52.705) (size 0.6) (drill 0.3) (layers "F.Cu" "B.Cu") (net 9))
 (via (at 125.095 70.104) (size 0.6) (drill 0.3) (layers "F.Cu" "B.Cu") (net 9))
 (via (at 103.124 61.468) (size 0.6) (drill 0.3) (layers "F.Cu" "B.Cu") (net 9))
 (via (at 127.254 62.103) (size 0.6) (drill 0.3) (layers "F.Cu" "B.Cu") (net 9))
 (via (at 122.174 54.102) (size 0.6) (drill 0.3) (layers "F.Cu" "B.Cu") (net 9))
 (via (at 105.537 71.755) (size 0.6) (drill 0.3) (layers "F.Cu" "B.Cu") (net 9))
 (segment (start 105.923 49.779) (end 102.997 52.705) (width 0.381) (layer "B.Cu") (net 9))
 (segment (start 114.554 49.779) (end 117.4775 52.7025) (width 0.381) (layer "B.Cu") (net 9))
 (segment (start 104.14 63.373) (end 104.785 64.018) (width 0.381) (layer "B.Cu") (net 9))
 (segment (start 122.489 70.485) (end 121.346 69.342) (width 0.381) (layer "B.Cu") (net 9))
 (segment (start 103.124 61.468) (end 103.124 62.357) (width 0.381) (layer "B.Cu") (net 9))
 (segment (start 117.4775 52.7025) (end 118.821 54.046) (width 0.381) (layer "B.Cu") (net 9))
 (segment (start 114.554 49.779) (end 111.6305 52.7025) (width 0.381) (layer "B.Cu") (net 9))
 (segment (start 124.968 65.278) (end 121.308 61.618) (width 0.381) (layer "B.Cu") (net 9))
 (segment (start 117.221 67.649) (end 117.221 66.518) (width 0.381) (layer "B.Cu") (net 9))
 (segment (start 117.972 49.779) (end 117.977 49.784) (width 0.381) (layer "B.Cu") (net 9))
 (segment (start 108.458 71.755) (end 105.537 71.755) (width 0.381) (layer "B.Cu") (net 9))
 (segment (start 127.254 62.992) (end 124.968 65.278) (width 0.381) (layer "B.Cu") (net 9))
 (segment (start 118.821 55.118) (end 121.158 55.118) (width 0.381) (layer "B.Cu") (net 9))
 (segment (start 104.785 64.018) (end 109.121 64.018) (width 0.381) (layer "B.Cu") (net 9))
 (segment (start 103.124 62.357) (end 104.14 63.373) (width 0.381) (layer "B.Cu") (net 9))
 (segment (start 111.6305 52.7025) (end 110.821 53.512) (width 0.381) (layer "B.Cu") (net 9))
 (segment (start 114.554 49.779) (end 105.923 49.779) (width 0.381) (layer "B.Cu") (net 9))
 (segment (start 118.914 69.342) (end 117.221 67.649) (width 0.381) (layer "B.Cu") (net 9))
 (segment (start 122.489 70.485) (end 124.714 70.485) (width 0.381) (layer "B.Cu") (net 9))
 (segment (start 110.821 53.512) (end 110.821 55.118) (width 0.381) (layer "B.Cu") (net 9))
 (segment (start 114.554 49.779) (end 117.972 49.779) (width 0.381) (layer "B.Cu") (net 9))
 (segment (start 118.821 54.046) (end 118.821 55.118) (width 0.381) (layer "B.Cu") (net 9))
 (segment (start 121.346 69.342) (end 118.914 69.342) (width 0.381) (layer "B.Cu") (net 9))
 (segment (start 121.158 55.118) (end 122.174 54.102) (width 0.381) (layer "B.Cu") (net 9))
 (segment (start 124.714 70.485) (end 125.095 70.104) (width 0.381) (layer "B.Cu") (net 9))
 (segment (start 127.254 62.103) (end 127.254 62.992) (width 0.381) (layer "B.Cu") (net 9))
 (segment (start 121.308 61.618) (end 120.521 61.618) (width 0.381) (layer "B.Cu") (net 9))
 (segment (start 114.821 73.079) (end 118.745 77.003) (width 0.254) (layer "B.Cu") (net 19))
 (segment (start 118.659 77.089) (end 118.745 77.003) (width 0.254) (layer "B.Cu") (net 19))
 (segment (start 113.46 77.089) (end 118.659 77.089) (width 0.254) (layer "B.Cu") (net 19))
 (segment (start 114.821 66.518) (end 114.821 73.079) (width 0.254) (layer "B.Cu") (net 19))
 (segment (start 115.621 69.879) (end 120.445 74.703) (width 0.254) (layer "B.Cu") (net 12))
 (segment (start 115.621 66.518) (end 115.621 69.879) (width 0.254) (layer "B.Cu") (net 12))
 (segment (start 120.826 75.184) (end 120.445 74.803) (width 0.254) (layer "B.Cu") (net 12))
 (segment (start 120.445 74.703) (end 120.445 74.803) (width 0.254) (layer "B.Cu") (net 12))
 (segment (start 125.779 75.184) (end 120.826 75.184) (width 0.254) (layer "B.Cu") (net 12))
 (segment (start 150.3269 52.69565) (end 150.01875 52.3875) (width 0.254) (layer "B.Cu") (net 46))
 (segment (start 169.06875 52.5125) (end 168.8856 52.69565) (width 0.254) (layer "B.Cu") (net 46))
 (segment (start 168.8856 52.69565) (end 150.3269 52.69565) (width 0.254) (layer "B.Cu") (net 46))
 (segment (start 144.4225 45.82375) (end 147.68625 49.0875) (width 0.254) (layer "B.Cu") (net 2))
 (segment (start 147.68625 49.0875) (end 150.01875 49.0875) (width 0.254) (layer "B.Cu") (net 2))
 (segment (start 166.86125 49.2125) (end 163.4725 45.82375) (width 0.254) (layer "B.Cu") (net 5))
 (segment (start 169.06875 49.2125) (end 166.86125 49.2125) (width 0.254) (layer "B.Cu") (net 5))
 (segment (start 144.402047 64.503178) (end 147.846928 64.503178) (width 0.254) (layer "B.Cu") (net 6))
 (segment (start 147.846928 64.503178) (end 150.01875 66.675) (width 0.254) (layer "B.Cu") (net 6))
 (segment (start 167.052755 71.990995) (end 152.034745 71.990995) (width 0.254) (layer "B.Cu") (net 15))
 (segment (start 152.034745 71.990995) (end 150.01875 69.975) (width 0.254) (layer "B.Cu") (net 15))
 (segment (start 169.06875 69.975) (end 167.052755 71.990995) (width 0.254) (layer "B.Cu") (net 15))
 (segment (start 164.98981 66.675) (end 169.06875 66.675) (width 0.254) (layer "B.Cu") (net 4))
 (segment (start 163.433905 65.119095) (end 164.98981 66.675) (width 0.254) (layer "B.Cu") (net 4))
 (segment (start 120.777 49.784) (end 122.299 49.784) (width 0.381) (layer "B.Cu") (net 11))
 (segment (start 122.299 49.784) (end 124.163 47.92) (width 0.381) (layer "B.Cu") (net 11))
 (segment (start 124.163 47.92) (end 124.163 47.045) (width 0.381) (layer "B.Cu") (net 11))
 (segment (start 108.395 56.092) (end 109.121 56.818) (width 0.254) (layer "B.Cu") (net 7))
 (segment (start 105.552 56.092) (end 108.395 56.092) (width 0.254) (layer "B.Cu") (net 7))
 (segment (start 125.603 52.959) (end 123.825 54.737) (width 0.254) (layer "B.Cu") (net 17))
 (segment (start 127.762 52.959) (end 125.603 52.959) (width 0.254) (layer "B.Cu") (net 17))
 (segment (start 128.016 52.705) (end 127.762 52.959) (width 0.254) (layer "B.Cu") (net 17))
 (segment (start 121.525 59.218) (end 120.521 59.218) (width 0.254) (layer "B.Cu") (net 17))
 (segment (start 123.825 54.737) (end 123.825 56.918) (width 0.254) (layer "B.Cu") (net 17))
 (segment (start 123.825 56.918) (end 121.525 59.218) (width 0.254) (layer "B.Cu") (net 17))
 (segment (start 127.461 50.88) (end 128.016 50.88) (width 0.2) (layer "B.Cu") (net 16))
 (segment (start 125.763 49.182) (end 127.461 50.88) (width 0.2) (layer "B.Cu") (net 16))
 (segment (start 125.763 47.045) (end 125.763 49.182) (width 0.2) (layer "B.Cu") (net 16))
 (segment (start 124.963 49.234) (end 123.317 50.88) (width 0.2) (layer "B.Cu") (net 13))
 (segment (start 124.963 47.045) (end 124.963 49.234) (width 0.2) (layer "B.Cu") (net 13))
 (segment (start 123.317 52.705) (end 123.317 56.626) (width 0.254) (layer "B.Cu") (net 14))
 (segment (start 121.525 58.418) (end 120.521 58.418) (width 0.254) (layer "B.Cu") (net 14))
 (segment (start 123.317 56.626) (end 121.525 58.418) (width 0.254) (layer "B.Cu") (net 14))
 (segment (start 119.634 68.199) (end 118.872 68.961) (width 0.254) (layer "F.Cu") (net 10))
 (segment (start 118.872 68.961) (end 112.014 68.961) (width 0.254) (layer "F.Cu") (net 10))
 (via (at 119.634 68.199) (size 0.6) (drill 0.3) (layers "F.Cu" "B.Cu") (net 10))
 (via (at 112.014 68.961) (size 0.6) (drill 0.3) (layers "F.Cu" "B.Cu") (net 10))
 (segment (start 107.754 74.284) (end 110.283 71.755) (width 0.254) (layer "B.Cu") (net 10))
 (segment (start 110.283 70.692) (end 112.014 68.961) (width 0.254) (layer "B.Cu") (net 10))
 (segment (start 99.083 73.406) (end 99.961 74.284) (width 0.254) (layer "B.Cu") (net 10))
 (segment (start 119.634 68.199) (end 118.999 68.199) (width 0.254) (layer "B.Cu") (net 10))
 (segment (start 99.961 74.284) (end 107.754 74.284) (width 0.254) (layer "B.Cu") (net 10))
 (segment (start 118.999 68.199) (end 118.021 67.221) (width 0.254) (layer "B.Cu") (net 10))
 (segment (start 118.021 67.221) (end 118.021 66.518) (width 0.254) (layer "B.Cu") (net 10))
 (segment (start 110.283 71.755) (end 110.283 70.692) (width 0.254) (layer "B.Cu") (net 10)))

